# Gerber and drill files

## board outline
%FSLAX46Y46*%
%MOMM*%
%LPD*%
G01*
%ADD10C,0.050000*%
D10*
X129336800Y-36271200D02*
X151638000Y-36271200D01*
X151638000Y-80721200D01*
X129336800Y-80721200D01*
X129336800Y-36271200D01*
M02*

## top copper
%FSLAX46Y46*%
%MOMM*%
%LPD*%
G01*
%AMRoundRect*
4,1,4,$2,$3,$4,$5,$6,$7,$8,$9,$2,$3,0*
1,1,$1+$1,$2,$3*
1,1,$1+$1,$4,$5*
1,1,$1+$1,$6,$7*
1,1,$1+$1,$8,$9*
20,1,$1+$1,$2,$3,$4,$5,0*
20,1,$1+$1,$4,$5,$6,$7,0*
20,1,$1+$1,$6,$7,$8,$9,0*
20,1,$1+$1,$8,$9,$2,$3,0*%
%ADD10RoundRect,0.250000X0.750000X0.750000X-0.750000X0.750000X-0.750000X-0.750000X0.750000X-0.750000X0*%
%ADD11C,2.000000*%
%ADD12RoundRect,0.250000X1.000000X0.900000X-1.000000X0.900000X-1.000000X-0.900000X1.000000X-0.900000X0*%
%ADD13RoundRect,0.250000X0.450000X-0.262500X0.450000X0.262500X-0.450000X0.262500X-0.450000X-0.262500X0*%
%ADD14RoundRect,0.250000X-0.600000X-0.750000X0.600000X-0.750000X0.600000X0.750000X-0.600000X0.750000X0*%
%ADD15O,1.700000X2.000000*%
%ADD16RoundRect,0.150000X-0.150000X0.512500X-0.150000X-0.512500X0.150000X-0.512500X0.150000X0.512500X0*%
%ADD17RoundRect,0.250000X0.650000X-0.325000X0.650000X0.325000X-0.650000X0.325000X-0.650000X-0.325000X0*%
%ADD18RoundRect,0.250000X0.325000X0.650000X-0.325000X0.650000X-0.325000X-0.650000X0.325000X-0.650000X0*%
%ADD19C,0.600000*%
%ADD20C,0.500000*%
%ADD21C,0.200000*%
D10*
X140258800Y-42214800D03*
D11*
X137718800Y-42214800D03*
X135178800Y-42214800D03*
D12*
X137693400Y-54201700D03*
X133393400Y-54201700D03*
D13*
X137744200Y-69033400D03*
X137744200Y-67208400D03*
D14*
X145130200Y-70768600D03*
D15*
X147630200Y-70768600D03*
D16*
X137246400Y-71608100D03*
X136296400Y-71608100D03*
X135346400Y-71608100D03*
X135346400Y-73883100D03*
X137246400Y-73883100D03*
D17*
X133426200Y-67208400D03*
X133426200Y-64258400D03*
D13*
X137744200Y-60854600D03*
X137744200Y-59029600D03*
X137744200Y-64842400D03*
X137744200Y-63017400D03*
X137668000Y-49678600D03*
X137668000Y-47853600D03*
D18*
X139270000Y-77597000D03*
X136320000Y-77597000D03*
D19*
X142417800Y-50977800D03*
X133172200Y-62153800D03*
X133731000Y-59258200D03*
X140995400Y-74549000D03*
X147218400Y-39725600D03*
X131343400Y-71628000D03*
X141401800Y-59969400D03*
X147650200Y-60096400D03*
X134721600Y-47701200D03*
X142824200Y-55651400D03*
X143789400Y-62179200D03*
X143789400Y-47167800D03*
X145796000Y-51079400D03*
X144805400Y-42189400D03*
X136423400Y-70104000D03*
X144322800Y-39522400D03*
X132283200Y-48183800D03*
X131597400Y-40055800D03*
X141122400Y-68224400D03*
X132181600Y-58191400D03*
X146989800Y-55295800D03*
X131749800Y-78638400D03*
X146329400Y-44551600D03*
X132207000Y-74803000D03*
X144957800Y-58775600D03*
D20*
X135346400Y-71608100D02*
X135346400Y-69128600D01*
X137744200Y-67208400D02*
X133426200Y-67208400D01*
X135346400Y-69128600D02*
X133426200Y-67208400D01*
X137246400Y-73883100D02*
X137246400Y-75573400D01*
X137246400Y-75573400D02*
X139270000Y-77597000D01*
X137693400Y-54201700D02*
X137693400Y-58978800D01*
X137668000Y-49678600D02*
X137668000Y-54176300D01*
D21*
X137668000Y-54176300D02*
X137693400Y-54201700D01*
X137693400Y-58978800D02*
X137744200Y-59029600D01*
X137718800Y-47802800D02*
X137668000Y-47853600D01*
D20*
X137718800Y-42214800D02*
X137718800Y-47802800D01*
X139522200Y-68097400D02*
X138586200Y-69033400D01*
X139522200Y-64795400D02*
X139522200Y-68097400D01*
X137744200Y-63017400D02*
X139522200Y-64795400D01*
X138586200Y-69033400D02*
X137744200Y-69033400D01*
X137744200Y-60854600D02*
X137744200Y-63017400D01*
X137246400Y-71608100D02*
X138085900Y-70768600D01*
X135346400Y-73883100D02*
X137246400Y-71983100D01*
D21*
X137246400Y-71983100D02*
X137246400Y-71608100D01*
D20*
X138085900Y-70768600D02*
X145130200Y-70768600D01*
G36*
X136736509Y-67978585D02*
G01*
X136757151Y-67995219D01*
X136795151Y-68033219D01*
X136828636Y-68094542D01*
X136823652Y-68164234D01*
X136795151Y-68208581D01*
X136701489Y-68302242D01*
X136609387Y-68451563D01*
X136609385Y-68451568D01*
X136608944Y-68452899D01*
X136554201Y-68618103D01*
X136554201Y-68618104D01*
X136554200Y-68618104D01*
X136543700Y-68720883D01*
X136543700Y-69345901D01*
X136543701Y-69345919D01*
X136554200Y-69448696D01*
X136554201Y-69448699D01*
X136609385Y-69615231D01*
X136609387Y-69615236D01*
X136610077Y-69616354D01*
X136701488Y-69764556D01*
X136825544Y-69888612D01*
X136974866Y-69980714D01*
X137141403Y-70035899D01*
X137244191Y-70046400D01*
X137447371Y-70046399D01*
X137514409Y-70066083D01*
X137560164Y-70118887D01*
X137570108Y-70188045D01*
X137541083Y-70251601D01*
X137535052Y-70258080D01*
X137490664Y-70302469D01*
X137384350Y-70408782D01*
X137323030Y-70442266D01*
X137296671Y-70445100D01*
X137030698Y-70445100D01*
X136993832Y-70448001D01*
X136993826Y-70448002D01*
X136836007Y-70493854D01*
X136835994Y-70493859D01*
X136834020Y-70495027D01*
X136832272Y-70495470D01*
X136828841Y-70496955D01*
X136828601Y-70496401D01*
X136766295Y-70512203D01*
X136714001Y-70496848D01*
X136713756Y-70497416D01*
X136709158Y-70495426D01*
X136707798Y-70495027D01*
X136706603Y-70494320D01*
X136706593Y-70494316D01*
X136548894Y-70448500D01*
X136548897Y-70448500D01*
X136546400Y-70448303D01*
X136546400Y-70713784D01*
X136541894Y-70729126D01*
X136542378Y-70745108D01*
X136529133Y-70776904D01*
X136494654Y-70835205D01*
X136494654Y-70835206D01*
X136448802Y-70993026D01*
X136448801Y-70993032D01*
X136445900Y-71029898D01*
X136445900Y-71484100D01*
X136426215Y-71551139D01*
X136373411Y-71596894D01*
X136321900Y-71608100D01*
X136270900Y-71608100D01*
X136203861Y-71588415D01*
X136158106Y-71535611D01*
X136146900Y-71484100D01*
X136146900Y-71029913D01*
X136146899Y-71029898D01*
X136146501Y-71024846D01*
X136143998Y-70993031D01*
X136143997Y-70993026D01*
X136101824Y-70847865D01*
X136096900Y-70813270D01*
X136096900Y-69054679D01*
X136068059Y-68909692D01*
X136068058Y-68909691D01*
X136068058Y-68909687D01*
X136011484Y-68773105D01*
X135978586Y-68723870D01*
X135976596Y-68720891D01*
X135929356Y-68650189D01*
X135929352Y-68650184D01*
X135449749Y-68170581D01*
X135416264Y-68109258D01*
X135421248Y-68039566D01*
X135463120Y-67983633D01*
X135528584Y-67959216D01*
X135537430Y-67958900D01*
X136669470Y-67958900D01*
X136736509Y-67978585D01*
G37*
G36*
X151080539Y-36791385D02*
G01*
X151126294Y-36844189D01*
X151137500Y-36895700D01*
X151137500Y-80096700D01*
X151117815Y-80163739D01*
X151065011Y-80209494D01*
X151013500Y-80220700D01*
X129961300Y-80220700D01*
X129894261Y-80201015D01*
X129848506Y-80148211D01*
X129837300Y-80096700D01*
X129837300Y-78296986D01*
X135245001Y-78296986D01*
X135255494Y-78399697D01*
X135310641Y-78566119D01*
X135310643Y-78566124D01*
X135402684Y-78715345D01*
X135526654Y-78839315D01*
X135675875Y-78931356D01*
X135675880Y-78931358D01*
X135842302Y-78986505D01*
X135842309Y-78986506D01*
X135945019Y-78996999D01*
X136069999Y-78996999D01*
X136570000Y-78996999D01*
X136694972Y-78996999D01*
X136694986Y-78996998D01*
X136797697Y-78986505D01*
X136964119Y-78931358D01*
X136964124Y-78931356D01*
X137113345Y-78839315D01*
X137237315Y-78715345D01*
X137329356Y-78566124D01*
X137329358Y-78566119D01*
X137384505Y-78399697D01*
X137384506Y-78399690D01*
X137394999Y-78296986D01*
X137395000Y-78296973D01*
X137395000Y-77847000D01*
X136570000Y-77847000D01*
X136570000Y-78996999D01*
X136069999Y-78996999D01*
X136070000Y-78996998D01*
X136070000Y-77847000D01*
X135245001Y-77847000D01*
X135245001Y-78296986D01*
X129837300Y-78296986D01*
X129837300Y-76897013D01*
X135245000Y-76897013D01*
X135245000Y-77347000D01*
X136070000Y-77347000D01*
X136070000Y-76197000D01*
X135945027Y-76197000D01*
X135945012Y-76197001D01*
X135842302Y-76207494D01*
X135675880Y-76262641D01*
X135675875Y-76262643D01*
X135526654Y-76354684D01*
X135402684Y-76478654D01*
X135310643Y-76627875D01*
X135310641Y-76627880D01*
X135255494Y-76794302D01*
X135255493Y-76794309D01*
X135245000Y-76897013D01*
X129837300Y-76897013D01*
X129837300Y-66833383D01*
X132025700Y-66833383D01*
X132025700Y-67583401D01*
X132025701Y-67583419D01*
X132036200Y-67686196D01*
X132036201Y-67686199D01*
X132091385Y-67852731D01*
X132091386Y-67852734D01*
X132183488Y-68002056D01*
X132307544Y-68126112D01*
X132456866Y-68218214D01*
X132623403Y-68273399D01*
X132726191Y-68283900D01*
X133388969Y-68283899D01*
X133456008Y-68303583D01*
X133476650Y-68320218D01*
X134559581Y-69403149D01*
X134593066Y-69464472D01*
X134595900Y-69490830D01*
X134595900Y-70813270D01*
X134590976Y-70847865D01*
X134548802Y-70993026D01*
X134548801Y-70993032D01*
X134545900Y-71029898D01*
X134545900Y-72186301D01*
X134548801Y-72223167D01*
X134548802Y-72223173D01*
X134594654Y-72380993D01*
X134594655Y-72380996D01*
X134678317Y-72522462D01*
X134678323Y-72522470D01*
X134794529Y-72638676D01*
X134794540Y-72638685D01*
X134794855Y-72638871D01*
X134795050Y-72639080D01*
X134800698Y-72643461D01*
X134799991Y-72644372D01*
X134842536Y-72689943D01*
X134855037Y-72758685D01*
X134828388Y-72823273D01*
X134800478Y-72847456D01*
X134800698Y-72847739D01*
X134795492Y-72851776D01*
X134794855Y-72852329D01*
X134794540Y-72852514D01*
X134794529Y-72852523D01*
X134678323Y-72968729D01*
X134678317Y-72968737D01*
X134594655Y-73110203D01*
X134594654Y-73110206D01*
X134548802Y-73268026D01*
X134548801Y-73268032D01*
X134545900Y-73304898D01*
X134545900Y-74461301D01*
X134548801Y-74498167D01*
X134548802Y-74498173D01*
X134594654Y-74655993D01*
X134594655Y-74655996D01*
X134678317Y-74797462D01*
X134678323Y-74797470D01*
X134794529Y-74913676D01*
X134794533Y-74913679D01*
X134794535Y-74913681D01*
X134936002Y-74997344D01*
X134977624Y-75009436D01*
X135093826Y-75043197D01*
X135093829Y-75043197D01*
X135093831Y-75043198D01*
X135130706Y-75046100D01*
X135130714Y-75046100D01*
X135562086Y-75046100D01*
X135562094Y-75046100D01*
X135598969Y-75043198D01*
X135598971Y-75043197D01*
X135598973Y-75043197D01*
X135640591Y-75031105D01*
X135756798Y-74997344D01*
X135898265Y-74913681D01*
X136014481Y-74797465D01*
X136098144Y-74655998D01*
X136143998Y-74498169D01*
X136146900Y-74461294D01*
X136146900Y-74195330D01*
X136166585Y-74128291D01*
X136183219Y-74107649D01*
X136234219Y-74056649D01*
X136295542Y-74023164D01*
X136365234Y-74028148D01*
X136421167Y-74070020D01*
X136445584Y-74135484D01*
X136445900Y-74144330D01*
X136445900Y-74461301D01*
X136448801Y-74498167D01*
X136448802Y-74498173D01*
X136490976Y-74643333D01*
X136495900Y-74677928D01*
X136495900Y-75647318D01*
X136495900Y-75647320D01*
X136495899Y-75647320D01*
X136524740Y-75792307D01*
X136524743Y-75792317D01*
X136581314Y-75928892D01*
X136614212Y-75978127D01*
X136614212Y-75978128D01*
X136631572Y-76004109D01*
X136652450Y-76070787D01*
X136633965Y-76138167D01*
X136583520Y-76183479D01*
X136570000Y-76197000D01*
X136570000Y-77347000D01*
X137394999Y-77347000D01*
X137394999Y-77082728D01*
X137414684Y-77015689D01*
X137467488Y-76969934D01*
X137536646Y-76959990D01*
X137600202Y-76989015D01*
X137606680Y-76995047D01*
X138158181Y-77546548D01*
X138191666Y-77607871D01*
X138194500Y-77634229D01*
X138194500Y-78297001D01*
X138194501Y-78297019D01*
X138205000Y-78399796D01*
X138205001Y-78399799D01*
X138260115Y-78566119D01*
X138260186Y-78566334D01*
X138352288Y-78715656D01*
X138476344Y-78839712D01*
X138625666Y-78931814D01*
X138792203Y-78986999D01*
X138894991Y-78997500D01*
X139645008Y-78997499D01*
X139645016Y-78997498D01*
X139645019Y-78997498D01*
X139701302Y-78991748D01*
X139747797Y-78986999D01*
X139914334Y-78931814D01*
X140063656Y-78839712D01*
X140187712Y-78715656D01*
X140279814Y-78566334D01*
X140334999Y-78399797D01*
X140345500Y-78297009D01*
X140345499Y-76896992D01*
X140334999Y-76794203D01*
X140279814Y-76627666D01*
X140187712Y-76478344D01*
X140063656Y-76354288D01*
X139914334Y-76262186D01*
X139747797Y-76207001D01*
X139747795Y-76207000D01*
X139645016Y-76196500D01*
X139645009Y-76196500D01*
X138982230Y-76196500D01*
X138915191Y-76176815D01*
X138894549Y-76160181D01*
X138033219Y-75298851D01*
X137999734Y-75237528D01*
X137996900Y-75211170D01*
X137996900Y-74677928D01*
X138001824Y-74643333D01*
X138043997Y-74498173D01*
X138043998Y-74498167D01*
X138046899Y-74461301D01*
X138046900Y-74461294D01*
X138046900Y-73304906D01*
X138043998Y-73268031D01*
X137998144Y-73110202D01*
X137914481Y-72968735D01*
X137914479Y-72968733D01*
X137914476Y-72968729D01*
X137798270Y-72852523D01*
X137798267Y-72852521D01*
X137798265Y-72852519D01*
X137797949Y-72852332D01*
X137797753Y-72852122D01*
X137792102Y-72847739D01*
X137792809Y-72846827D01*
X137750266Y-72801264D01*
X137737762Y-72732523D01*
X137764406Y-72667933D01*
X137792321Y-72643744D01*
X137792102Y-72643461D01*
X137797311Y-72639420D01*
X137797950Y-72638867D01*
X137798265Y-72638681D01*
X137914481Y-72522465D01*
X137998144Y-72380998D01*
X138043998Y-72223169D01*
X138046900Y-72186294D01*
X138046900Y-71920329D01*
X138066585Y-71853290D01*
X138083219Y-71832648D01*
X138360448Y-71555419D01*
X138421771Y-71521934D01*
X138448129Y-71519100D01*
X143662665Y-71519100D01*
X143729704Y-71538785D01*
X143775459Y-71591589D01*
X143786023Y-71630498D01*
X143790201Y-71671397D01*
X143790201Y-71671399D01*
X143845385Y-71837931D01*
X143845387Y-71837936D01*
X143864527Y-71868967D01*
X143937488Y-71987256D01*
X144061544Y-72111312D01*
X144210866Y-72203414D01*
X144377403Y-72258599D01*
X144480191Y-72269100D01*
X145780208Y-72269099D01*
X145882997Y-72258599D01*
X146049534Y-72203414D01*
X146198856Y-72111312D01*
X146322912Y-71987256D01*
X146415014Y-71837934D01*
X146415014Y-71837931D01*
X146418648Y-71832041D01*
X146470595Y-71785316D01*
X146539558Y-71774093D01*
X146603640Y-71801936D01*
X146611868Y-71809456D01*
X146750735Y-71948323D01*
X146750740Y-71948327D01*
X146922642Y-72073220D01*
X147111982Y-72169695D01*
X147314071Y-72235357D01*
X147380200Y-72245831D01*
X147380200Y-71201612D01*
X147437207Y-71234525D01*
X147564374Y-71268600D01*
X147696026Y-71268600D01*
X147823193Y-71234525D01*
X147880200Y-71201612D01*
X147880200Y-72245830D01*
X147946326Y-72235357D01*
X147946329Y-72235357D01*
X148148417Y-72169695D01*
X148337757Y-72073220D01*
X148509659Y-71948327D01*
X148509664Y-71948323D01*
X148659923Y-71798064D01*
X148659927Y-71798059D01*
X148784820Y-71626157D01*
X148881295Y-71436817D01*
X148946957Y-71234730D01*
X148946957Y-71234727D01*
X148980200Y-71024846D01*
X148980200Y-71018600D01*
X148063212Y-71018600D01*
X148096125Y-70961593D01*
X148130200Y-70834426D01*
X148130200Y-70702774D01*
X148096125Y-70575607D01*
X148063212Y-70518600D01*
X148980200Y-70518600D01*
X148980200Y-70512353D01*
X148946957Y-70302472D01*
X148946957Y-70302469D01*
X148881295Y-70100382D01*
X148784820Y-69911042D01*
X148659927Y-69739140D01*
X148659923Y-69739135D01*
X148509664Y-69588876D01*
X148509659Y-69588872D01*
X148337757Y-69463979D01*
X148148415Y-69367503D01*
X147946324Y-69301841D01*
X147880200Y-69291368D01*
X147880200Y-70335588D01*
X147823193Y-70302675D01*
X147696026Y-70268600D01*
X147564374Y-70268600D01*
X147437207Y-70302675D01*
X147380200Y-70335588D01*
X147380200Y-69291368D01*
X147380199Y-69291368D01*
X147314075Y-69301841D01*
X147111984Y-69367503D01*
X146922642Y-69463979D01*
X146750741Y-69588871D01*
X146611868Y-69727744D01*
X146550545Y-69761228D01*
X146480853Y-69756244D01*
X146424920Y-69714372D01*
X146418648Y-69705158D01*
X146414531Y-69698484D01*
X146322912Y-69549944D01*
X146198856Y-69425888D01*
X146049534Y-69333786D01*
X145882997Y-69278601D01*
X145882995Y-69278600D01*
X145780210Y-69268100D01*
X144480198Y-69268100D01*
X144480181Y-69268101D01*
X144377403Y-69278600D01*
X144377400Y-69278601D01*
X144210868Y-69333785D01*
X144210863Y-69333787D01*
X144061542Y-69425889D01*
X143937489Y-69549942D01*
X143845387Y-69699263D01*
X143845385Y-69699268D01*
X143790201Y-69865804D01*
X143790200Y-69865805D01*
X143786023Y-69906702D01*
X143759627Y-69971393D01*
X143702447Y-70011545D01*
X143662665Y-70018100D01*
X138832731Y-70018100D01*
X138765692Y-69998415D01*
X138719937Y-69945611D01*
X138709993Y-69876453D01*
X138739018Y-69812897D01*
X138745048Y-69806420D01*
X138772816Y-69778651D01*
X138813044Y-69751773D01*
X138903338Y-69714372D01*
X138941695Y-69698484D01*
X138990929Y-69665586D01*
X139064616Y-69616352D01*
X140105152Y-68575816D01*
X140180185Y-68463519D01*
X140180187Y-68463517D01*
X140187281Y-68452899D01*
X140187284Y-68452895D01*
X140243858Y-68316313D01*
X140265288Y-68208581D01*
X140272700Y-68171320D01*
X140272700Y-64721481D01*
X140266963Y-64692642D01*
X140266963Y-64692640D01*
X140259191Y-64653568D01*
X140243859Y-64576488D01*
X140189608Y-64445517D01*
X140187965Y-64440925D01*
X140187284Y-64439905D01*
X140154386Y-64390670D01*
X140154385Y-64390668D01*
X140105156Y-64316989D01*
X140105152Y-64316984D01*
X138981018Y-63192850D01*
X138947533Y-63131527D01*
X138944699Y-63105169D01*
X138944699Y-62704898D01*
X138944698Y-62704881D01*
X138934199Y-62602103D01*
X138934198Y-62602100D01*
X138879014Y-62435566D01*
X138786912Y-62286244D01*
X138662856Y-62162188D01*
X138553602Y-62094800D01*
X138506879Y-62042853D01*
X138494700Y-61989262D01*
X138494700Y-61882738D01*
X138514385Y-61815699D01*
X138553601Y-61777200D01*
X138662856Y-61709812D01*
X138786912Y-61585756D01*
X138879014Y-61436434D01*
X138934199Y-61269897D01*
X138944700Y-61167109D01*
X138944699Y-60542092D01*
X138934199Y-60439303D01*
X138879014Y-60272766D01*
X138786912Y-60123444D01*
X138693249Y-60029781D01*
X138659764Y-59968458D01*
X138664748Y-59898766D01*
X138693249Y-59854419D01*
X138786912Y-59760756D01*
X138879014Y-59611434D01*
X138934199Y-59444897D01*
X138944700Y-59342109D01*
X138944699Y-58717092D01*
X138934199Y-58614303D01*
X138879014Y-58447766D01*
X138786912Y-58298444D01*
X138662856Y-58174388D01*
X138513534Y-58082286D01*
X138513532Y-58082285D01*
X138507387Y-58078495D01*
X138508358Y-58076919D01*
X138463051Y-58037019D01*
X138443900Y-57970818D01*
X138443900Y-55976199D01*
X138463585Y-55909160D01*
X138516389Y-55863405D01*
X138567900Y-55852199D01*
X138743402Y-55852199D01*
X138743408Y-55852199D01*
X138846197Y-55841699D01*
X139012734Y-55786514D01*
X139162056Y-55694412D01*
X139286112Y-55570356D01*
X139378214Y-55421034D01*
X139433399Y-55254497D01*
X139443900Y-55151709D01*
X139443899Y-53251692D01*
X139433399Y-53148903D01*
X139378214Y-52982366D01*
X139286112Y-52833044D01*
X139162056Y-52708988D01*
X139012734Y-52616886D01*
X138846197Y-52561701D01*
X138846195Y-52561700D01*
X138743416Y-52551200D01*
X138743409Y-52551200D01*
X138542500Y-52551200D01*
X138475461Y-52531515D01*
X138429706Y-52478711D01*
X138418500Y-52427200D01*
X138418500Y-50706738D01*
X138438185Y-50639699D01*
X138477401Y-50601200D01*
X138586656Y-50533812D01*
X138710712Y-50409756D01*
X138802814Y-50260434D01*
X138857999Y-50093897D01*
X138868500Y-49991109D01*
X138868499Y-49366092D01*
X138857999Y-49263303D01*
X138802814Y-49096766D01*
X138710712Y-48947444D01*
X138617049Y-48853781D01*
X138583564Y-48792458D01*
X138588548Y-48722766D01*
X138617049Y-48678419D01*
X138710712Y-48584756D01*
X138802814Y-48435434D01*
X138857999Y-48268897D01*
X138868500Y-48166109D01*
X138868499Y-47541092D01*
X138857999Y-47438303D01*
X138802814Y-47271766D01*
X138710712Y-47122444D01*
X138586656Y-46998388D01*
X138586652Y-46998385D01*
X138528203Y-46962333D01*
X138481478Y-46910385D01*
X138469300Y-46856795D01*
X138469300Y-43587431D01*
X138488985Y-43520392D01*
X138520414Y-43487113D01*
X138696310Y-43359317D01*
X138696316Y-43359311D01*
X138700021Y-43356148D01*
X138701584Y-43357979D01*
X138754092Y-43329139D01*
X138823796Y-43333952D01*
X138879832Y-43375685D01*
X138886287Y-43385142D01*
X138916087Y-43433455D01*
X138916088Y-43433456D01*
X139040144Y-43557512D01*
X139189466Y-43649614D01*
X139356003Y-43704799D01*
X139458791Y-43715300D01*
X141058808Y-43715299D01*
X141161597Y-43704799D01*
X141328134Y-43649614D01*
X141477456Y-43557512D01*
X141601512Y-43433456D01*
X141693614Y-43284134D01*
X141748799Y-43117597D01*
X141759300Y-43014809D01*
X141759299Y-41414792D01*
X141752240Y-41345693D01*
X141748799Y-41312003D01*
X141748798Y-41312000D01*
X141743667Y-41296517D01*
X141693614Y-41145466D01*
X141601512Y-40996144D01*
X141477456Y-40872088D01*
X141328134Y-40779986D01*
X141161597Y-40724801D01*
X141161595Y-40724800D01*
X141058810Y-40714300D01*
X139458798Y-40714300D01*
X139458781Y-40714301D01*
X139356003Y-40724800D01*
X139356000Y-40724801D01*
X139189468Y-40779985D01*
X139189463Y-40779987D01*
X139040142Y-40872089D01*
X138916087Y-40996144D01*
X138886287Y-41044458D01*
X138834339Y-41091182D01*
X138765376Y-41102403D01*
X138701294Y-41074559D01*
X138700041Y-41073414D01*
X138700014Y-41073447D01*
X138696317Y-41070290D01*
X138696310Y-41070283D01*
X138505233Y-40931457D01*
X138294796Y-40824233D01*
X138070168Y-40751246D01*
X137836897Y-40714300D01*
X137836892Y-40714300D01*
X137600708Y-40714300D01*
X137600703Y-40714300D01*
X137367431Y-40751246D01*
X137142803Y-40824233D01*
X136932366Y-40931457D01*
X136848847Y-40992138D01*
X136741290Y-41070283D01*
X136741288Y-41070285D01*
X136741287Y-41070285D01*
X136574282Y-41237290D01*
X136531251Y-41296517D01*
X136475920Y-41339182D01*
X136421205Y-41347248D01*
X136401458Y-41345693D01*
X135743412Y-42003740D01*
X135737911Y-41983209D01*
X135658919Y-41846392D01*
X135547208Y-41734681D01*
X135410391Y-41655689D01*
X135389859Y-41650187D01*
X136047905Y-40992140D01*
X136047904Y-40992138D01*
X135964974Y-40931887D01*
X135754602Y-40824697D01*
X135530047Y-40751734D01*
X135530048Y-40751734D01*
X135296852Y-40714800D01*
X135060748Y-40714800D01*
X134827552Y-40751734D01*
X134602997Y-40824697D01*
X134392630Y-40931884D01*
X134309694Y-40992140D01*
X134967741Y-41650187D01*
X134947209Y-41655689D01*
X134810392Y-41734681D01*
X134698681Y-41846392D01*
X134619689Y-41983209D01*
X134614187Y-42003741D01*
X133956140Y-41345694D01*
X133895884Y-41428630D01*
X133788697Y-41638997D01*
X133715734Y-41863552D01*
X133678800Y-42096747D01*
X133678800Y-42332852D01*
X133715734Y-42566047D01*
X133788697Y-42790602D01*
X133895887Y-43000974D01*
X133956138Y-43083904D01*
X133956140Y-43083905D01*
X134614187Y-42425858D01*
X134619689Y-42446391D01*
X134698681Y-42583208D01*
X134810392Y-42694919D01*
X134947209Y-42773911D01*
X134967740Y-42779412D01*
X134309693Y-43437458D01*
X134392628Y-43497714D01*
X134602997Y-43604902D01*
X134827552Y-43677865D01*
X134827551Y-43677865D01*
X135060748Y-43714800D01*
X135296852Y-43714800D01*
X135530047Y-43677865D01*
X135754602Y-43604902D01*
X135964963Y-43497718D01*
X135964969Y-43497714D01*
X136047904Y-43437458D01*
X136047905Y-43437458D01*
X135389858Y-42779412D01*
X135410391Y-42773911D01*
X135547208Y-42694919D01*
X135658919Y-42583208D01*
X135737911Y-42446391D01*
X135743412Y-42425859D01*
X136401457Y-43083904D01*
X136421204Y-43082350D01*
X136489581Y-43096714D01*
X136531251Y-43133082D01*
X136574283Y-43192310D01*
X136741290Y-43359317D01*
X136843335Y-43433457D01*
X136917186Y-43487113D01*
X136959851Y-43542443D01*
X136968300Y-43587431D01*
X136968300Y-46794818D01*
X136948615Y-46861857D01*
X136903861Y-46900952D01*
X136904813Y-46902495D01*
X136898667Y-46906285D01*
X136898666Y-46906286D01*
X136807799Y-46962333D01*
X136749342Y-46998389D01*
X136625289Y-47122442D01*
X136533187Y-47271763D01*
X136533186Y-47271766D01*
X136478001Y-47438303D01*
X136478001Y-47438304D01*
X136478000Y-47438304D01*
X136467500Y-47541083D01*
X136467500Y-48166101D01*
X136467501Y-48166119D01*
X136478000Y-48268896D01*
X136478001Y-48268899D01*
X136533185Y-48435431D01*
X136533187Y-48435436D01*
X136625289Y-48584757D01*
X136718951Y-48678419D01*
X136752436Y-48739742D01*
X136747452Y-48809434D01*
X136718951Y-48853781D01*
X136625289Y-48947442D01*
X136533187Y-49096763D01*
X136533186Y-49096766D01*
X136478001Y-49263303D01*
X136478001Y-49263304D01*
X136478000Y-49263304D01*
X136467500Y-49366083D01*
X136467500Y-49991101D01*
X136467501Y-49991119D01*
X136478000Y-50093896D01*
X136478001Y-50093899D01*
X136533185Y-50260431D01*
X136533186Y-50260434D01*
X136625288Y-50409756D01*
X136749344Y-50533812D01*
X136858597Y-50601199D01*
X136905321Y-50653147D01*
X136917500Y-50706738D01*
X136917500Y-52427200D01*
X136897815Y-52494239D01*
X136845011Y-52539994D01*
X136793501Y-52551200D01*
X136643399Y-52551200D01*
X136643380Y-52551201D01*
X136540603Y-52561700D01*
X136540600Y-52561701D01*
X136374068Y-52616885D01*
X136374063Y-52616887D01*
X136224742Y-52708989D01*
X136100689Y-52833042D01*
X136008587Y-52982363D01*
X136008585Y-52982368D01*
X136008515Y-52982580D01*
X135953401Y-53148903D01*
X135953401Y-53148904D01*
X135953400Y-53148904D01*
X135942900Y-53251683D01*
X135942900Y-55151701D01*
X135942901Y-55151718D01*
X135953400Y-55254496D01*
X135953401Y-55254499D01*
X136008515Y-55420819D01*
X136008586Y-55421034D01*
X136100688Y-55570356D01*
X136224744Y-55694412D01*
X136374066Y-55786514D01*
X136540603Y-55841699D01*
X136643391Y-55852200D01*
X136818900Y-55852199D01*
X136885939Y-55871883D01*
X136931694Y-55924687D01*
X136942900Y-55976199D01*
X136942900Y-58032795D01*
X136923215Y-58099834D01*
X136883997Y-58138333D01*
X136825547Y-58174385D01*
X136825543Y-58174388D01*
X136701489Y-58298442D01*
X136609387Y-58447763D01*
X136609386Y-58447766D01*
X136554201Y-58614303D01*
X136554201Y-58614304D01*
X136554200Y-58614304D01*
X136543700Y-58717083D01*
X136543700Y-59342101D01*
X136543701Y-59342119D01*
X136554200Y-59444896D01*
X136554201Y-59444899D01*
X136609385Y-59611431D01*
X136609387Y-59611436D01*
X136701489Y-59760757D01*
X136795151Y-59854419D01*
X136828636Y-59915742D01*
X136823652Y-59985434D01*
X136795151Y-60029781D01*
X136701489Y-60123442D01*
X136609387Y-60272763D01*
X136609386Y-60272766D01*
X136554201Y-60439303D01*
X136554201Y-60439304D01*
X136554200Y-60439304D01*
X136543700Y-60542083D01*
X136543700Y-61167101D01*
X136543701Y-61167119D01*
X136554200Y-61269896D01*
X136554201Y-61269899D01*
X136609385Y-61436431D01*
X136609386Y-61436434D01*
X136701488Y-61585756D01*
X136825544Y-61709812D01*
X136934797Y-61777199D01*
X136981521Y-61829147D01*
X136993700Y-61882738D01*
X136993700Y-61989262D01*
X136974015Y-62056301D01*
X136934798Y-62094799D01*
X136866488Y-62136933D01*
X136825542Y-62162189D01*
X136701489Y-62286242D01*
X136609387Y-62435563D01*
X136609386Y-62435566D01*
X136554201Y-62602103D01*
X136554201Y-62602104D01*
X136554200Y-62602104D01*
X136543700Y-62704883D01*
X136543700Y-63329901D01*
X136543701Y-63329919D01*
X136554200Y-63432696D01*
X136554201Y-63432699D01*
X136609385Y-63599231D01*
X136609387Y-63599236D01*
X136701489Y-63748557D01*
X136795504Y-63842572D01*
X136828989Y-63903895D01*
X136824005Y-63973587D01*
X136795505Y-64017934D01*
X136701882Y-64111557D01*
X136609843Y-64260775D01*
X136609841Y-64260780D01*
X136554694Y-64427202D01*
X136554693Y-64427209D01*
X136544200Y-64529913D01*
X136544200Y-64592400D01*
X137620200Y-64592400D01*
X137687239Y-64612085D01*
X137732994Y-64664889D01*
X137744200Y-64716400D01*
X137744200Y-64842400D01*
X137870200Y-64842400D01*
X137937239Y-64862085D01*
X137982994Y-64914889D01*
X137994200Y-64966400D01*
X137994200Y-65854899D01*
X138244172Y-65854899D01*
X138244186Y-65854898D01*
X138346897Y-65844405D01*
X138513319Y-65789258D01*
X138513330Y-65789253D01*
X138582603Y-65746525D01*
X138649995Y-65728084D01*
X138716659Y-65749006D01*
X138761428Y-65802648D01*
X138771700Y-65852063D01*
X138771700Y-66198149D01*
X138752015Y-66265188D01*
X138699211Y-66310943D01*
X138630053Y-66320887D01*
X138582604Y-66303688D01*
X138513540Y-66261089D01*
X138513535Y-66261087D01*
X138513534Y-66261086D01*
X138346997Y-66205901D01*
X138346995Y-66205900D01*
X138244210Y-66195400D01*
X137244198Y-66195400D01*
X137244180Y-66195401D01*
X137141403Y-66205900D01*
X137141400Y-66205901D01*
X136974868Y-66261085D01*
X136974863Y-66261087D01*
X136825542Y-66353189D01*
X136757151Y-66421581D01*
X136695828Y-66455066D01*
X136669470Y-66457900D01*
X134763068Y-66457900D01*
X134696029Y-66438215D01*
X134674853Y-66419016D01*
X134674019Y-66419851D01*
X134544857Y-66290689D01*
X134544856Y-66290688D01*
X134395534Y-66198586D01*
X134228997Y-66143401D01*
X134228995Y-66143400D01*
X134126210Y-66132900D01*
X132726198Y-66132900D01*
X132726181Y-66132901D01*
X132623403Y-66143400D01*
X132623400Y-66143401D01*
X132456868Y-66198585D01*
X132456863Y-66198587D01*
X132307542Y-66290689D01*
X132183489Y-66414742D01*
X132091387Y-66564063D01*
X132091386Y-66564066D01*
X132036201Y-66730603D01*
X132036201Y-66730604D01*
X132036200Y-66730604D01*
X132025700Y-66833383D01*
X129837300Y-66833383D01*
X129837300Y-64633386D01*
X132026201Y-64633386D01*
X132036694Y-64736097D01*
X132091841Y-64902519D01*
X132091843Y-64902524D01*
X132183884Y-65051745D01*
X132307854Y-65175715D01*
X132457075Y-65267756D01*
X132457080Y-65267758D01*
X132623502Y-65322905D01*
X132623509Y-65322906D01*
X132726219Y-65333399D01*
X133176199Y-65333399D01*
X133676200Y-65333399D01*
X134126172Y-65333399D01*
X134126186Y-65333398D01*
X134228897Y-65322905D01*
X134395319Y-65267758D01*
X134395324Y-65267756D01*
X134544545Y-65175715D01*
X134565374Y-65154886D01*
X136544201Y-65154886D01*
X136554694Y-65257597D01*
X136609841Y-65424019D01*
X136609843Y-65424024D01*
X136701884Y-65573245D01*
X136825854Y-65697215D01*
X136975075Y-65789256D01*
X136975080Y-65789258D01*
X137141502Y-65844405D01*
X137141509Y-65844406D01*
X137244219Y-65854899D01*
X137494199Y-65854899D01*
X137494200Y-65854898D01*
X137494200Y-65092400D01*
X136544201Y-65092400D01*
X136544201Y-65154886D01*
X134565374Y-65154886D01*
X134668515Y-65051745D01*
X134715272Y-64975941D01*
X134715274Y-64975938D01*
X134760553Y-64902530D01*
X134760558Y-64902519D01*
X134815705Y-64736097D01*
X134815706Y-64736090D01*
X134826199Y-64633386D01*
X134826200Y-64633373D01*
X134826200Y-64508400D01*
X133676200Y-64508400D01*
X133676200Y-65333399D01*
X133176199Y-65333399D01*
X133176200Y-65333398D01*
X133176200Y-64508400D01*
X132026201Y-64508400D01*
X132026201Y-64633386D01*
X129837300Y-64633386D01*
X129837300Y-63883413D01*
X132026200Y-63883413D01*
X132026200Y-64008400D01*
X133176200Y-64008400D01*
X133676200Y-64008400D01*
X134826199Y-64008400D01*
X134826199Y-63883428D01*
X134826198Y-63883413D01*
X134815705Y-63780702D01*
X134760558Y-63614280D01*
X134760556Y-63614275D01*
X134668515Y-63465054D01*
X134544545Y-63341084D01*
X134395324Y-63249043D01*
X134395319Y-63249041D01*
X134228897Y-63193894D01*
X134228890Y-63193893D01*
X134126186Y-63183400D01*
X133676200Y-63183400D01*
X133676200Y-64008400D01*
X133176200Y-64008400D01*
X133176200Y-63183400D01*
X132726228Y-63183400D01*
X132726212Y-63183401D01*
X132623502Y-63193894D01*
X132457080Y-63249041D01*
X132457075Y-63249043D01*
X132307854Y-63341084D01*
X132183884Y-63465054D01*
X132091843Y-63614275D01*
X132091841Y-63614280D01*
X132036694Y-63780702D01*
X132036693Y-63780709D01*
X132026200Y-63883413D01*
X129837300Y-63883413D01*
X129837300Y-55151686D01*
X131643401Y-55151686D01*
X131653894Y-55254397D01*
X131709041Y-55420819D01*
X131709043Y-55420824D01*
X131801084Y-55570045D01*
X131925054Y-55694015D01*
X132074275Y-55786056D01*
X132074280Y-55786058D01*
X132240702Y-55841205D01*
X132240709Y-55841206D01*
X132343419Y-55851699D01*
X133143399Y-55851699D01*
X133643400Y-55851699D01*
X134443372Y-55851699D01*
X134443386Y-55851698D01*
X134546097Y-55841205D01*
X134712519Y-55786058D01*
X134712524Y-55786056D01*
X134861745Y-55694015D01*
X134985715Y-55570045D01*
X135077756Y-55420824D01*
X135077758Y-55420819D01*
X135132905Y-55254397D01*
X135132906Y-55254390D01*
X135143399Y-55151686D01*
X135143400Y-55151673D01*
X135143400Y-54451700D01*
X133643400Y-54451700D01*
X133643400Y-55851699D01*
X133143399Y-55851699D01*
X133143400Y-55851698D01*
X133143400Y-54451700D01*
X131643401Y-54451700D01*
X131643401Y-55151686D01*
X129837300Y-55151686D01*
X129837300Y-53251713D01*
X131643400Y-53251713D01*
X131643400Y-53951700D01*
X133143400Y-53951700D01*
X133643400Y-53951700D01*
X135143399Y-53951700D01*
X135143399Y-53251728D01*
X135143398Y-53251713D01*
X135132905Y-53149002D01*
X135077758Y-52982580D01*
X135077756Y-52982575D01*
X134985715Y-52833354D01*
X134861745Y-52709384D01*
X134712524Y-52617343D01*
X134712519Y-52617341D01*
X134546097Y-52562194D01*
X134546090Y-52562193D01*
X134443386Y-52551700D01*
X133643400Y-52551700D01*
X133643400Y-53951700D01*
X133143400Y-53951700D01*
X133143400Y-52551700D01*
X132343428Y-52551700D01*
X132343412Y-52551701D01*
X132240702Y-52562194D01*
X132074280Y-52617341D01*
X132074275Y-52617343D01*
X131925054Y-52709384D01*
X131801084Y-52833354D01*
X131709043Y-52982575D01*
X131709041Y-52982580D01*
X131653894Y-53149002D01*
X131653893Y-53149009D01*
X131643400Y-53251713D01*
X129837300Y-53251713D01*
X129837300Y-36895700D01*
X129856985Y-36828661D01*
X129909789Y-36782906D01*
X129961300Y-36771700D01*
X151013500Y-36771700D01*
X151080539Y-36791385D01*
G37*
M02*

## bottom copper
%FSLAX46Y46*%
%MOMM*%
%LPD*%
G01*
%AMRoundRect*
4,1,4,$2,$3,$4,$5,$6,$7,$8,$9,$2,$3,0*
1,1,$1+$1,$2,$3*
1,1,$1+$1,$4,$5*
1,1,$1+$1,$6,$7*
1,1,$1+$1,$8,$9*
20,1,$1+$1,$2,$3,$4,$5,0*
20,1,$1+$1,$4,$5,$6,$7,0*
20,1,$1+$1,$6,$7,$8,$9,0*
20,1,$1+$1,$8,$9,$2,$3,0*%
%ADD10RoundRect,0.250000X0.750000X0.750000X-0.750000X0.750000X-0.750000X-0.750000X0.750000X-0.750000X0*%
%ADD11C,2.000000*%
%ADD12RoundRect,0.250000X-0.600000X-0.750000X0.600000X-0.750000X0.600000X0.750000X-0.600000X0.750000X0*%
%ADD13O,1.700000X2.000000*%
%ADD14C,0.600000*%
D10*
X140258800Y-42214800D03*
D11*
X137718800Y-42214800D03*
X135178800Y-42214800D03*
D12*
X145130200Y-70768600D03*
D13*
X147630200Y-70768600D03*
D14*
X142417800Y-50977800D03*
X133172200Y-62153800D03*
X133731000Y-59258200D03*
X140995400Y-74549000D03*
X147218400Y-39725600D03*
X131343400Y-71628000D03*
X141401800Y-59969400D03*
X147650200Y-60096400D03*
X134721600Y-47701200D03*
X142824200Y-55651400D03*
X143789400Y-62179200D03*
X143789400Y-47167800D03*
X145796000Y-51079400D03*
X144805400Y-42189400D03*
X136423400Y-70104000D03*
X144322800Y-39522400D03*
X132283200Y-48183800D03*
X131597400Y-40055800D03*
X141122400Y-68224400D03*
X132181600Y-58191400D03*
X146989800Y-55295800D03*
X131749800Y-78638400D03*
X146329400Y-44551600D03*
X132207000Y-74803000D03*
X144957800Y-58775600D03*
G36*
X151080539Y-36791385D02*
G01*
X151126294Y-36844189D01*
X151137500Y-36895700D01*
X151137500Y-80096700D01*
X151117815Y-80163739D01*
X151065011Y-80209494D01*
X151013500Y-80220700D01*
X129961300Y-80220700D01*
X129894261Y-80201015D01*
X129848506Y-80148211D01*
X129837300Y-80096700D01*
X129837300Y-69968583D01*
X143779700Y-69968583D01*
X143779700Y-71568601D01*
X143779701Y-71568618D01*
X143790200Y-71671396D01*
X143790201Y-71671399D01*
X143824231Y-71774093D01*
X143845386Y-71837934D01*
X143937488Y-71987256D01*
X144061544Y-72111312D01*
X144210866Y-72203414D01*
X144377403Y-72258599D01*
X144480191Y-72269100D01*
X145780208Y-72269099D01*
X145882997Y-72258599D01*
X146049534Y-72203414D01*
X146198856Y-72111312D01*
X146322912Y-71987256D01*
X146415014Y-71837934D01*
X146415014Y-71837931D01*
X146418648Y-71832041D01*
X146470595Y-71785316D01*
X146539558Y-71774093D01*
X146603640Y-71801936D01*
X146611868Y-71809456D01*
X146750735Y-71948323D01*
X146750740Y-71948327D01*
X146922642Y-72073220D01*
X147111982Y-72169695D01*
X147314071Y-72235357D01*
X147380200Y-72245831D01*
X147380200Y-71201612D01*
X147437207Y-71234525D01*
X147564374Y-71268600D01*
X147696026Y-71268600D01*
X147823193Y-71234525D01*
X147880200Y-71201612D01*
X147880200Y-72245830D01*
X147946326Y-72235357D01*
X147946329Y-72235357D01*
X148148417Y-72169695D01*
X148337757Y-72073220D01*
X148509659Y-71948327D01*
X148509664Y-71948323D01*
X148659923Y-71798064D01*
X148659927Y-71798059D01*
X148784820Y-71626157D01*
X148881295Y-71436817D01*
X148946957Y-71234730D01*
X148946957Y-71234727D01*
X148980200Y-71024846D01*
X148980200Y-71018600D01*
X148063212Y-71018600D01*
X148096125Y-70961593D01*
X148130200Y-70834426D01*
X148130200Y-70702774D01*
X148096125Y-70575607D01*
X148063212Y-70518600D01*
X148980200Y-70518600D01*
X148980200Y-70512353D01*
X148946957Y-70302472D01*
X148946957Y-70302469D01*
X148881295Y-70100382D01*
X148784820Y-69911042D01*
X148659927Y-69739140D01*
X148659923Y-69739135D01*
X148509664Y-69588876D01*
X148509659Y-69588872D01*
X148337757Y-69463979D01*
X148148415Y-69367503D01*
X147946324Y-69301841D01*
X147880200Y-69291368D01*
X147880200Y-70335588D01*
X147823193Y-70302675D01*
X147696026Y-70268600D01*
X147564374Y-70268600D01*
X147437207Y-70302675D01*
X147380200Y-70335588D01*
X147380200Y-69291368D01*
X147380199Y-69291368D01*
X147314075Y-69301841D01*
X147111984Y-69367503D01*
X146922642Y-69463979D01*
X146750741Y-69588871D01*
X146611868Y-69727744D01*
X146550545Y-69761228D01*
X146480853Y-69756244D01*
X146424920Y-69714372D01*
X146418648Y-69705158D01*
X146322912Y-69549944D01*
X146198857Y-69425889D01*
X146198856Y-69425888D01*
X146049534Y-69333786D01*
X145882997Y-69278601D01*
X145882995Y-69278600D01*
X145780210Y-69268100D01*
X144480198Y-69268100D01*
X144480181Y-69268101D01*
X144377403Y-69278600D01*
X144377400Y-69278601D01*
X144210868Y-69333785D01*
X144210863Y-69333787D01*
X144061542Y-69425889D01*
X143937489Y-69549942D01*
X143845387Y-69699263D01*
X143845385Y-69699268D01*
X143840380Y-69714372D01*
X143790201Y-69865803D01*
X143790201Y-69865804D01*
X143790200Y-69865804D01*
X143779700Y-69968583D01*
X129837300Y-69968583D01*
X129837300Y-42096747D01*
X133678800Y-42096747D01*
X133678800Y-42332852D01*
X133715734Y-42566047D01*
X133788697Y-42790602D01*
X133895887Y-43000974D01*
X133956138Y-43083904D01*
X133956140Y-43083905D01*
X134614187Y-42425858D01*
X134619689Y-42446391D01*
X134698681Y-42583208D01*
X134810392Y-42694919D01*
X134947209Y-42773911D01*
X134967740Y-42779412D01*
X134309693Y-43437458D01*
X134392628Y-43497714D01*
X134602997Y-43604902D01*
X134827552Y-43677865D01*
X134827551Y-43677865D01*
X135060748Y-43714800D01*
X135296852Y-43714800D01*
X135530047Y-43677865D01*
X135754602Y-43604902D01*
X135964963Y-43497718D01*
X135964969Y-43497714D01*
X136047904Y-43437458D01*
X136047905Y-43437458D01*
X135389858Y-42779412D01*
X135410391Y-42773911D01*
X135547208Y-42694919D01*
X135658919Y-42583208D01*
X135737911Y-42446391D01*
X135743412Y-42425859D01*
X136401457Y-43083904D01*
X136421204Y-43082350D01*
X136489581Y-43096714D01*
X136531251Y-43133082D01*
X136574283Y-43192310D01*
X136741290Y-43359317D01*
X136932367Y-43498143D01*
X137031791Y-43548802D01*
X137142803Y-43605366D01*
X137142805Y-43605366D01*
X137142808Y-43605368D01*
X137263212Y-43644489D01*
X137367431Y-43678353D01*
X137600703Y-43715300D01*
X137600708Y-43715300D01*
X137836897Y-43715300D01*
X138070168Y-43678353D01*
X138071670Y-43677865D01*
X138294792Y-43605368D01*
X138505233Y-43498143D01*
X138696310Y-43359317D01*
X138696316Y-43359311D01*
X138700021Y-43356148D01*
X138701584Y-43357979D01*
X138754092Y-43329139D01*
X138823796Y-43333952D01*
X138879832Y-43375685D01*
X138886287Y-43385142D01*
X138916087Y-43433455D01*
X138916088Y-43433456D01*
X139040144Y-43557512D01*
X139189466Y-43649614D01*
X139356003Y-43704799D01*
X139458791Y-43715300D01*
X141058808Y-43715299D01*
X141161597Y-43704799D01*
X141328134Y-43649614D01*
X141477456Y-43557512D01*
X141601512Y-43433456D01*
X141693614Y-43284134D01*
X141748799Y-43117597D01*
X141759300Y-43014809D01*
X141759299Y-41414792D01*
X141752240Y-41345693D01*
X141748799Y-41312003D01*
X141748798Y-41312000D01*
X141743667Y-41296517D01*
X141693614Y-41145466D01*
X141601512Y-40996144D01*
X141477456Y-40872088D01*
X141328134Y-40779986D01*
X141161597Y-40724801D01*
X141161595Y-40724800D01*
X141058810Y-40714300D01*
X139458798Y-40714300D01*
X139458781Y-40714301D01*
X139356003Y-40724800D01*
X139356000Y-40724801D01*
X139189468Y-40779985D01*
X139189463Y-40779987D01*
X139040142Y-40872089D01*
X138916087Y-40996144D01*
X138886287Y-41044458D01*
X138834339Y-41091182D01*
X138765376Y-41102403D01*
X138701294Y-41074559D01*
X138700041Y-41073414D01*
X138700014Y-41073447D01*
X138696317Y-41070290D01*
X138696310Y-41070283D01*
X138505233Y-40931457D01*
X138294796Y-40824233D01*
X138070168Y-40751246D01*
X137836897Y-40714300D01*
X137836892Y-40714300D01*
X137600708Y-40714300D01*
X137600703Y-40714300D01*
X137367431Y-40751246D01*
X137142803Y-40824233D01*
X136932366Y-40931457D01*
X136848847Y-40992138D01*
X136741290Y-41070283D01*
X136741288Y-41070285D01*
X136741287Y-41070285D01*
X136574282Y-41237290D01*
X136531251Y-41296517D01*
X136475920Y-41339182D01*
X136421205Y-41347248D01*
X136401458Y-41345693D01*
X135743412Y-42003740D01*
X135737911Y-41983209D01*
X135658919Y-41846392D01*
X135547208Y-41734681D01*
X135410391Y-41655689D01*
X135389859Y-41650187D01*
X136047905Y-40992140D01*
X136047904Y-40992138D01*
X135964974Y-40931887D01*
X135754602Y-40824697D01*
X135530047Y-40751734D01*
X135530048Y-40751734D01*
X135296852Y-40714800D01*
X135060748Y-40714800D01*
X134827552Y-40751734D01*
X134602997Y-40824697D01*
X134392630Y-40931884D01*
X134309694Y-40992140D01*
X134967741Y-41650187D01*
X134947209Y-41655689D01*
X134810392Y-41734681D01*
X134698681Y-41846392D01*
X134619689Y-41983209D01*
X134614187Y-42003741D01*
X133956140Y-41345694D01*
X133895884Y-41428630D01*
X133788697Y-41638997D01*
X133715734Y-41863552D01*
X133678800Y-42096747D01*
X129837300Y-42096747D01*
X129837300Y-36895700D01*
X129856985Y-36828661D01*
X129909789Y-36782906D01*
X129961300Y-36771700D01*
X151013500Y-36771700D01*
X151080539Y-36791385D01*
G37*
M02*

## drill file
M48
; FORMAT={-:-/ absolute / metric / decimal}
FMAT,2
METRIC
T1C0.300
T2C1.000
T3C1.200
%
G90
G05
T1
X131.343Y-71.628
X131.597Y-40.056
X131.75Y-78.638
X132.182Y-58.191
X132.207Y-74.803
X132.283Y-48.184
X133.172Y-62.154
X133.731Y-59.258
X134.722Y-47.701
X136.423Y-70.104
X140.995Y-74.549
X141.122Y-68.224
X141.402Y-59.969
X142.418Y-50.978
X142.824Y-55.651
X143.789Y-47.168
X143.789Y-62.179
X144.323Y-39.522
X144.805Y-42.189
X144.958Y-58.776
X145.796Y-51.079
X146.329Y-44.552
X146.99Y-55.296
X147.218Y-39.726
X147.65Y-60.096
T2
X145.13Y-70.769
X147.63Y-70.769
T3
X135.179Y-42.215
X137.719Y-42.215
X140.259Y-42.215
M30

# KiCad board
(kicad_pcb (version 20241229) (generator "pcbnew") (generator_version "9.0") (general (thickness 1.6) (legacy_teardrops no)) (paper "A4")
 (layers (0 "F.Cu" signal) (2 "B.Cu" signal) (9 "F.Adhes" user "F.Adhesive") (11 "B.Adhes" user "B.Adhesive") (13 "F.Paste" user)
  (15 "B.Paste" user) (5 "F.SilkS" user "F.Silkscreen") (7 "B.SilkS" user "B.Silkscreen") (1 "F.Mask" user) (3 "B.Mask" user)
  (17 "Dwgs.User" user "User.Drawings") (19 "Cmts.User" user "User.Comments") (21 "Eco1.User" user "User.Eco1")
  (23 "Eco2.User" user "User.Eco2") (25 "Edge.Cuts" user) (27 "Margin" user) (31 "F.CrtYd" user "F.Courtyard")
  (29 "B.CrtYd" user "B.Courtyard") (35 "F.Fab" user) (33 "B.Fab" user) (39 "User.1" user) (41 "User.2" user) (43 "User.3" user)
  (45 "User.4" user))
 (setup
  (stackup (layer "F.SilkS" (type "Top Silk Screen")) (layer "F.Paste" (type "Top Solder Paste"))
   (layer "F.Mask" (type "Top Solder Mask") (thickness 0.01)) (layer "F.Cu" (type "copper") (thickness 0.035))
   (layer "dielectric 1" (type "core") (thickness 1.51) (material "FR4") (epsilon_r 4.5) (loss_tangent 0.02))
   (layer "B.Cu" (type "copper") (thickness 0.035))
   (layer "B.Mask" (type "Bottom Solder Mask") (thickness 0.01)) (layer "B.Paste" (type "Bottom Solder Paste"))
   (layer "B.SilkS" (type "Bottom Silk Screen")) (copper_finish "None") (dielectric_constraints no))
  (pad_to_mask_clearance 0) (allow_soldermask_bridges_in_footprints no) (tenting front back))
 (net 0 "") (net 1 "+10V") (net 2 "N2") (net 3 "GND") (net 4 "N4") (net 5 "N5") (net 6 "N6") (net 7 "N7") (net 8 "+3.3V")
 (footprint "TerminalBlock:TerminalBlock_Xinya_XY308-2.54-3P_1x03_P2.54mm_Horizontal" (layer "F.Cu") (at 140.2588 42.2148 180)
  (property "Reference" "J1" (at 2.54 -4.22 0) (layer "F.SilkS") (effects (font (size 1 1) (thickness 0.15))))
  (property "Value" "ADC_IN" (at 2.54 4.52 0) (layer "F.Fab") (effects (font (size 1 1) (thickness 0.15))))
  (pad "1" thru_hole roundrect (at 0 0 180) (size 2 2) (drill 1.2) (layers "*.Cu" "*.Mask") (remove_unused_layers no)
   (roundrect_rratio 0.125) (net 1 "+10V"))
  (pad "2" thru_hole circle (at 2.54 0 180) (size 2 2) (drill 1.2) (layers "*.Cu" "*.Mask") (remove_unused_layers no) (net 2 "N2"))
  (pad "3" thru_hole circle (at 5.08 0 180) (size 2 2) (drill 1.2) (layers "*.Cu" "*.Mask") (remove_unused_layers no) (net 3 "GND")))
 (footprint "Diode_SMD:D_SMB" (layer "F.Cu") (at 135.5434 54.2017 180)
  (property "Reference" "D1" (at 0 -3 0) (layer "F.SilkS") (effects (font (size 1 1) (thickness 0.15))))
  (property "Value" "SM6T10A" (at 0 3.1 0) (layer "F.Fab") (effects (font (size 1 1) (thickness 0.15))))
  (pad "1" smd roundrect (at -2.15 0 180) (size 2.5 2.3) (layers "F.Cu" "F.Mask" "F.Paste") (roundrect_rratio 0.1086956522) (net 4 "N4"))
  (pad "2" smd roundrect (at 2.15 0 180) (size 2.5 2.3) (layers "F.Cu" "F.Mask" "F.Paste") (roundrect_rratio 0.1086956522) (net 3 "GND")))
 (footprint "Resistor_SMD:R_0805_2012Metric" (layer "F.Cu") (at 137.7442 68.1209 90)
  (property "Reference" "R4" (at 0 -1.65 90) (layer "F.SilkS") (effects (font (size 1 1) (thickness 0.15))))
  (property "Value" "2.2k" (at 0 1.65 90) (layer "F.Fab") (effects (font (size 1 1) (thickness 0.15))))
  (pad "1" smd roundrect (at -0.9125 0 90) (size 1.025 1.4) (layers "F.Cu" "F.Mask" "F.Paste") (roundrect_rratio 0.243902) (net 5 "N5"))
  (pad "2" smd roundrect (at 0.9125 0 90) (size 1.025 1.4) (layers "F.Cu" "F.Mask" "F.Paste") (roundrect_rratio 0.243902) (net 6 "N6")))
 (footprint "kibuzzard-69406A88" (layer "F.Cu") (at 149.8346 46.2788 90)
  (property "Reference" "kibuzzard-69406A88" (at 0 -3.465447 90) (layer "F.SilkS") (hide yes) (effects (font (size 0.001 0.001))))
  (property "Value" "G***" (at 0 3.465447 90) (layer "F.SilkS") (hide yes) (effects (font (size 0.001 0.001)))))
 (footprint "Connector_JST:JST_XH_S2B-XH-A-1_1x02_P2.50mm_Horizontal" (layer "F.Cu") (at 145.1302 70.7686)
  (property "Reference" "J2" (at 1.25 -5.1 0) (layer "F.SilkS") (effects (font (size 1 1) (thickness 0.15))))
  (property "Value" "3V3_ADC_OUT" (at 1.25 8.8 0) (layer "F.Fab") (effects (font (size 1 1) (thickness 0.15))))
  (pad "1" thru_hole roundrect (at 0 0) (size 1.7 2) (drill 1) (layers "*.Cu" "*.Mask") (remove_unused_layers no)
   (roundrect_rratio 0.147059) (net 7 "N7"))
  (pad "2" thru_hole oval (at 2.5 0) (size 1.7 2) (drill 1) (layers "*.Cu" "*.Mask") (remove_unused_layers no) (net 3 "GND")))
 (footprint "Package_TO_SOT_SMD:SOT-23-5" (layer "F.Cu") (at 136.2964 72.7456 -90)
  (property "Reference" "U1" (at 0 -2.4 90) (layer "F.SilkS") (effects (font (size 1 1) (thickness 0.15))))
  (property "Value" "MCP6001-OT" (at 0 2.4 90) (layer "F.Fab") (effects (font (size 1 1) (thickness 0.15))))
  (pad "1" smd roundrect (at -1.1375 -0.95 270) (size 1.325 0.6) (layers "F.Cu" "F.Mask" "F.Paste") (roundrect_rratio 0.25) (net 7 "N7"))
  (pad "2" smd roundrect (at -1.1375 0 270) (size 1.325 0.6) (layers "F.Cu" "F.Mask" "F.Paste") (roundrect_rratio 0.25) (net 3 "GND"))
  (pad "3" smd roundrect (at -1.1375 0.95 270) (size 1.325 0.6) (layers "F.Cu" "F.Mask" "F.Paste") (roundrect_rratio 0.25) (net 6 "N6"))
  (pad "4" smd roundrect (at 1.1375 0.95 270) (size 1.325 0.6) (layers "F.Cu" "F.Mask" "F.Paste") (roundrect_rratio 0.25) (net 7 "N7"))
  (pad "5" smd roundrect (at 1.1375 -0.95 270) (size 1.325 0.6) (layers "F.Cu" "F.Mask" "F.Paste") (roundrect_rratio 0.25) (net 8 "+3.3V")))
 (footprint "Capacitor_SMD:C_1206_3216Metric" (layer "F.Cu") (at 133.4262 65.7334 90)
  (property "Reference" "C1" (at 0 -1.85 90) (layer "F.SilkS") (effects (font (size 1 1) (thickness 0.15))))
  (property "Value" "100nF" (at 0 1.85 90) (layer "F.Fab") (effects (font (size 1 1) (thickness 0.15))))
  (pad "1" smd roundrect (at -1.475 0 90) (size 1.15 1.8) (layers "F.Cu" "F.Mask" "F.Paste") (roundrect_rratio 0.217391) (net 6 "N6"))
  (pad "2" smd roundrect (at 1.475 0 90) (size 1.15 1.8) (layers "F.Cu" "F.Mask" "F.Paste") (roundrect_rratio 0.217391) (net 3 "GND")))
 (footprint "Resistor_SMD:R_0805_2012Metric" (layer "F.Cu") (at 137.7442 59.9421 90)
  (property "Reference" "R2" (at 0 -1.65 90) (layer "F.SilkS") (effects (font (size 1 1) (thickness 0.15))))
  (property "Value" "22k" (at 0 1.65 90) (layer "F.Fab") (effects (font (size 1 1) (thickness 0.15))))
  (pad "1" smd roundrect (at -0.9125 0 90) (size 1.025 1.4) (layers "F.Cu" "F.Mask" "F.Paste") (roundrect_rratio 0.243902) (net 5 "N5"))
  (pad "2" smd roundrect (at 0.9125 0 90) (size 1.025 1.4) (layers "F.Cu" "F.Mask" "F.Paste") (roundrect_rratio 0.243902) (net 4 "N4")))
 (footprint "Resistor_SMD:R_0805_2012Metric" (layer "F.Cu") (at 137.7442 63.9299 90)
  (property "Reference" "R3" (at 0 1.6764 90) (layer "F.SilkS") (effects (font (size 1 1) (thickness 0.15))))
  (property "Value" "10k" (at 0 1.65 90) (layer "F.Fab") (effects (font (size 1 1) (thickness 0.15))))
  (pad "1" smd roundrect (at -0.9125 0 90) (size 1.025 1.4) (layers "F.Cu" "F.Mask" "F.Paste") (roundrect_rratio 0.243902) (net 3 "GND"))
  (pad "2" smd roundrect (at 0.9125 0 90) (size 1.025 1.4) (layers "F.Cu" "F.Mask" "F.Paste") (roundrect_rratio 0.243902) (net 5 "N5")))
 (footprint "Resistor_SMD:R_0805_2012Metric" (layer "F.Cu") (at 137.668 48.7661 90)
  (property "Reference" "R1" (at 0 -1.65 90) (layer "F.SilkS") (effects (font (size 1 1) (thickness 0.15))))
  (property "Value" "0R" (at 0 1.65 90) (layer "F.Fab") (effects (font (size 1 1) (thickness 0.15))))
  (pad "1" smd roundrect (at -0.9125 0 90) (size 1.025 1.4) (layers "F.Cu" "F.Mask" "F.Paste") (roundrect_rratio 0.243902) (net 4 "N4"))
  (pad "2" smd roundrect (at 0.9125 0 90) (size 1.025 1.4) (layers "F.Cu" "F.Mask" "F.Paste") (roundrect_rratio 0.243902) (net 2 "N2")))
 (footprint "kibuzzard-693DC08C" (layer "F.Cu") (at 140.2842 37.2872 180)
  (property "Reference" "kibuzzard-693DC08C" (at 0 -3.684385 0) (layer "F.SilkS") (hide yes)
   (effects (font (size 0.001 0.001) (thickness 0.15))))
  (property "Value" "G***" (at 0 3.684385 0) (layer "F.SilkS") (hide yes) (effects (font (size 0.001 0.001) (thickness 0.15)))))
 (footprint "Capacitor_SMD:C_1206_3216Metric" (layer "F.Cu") (at 137.795 77.597 180)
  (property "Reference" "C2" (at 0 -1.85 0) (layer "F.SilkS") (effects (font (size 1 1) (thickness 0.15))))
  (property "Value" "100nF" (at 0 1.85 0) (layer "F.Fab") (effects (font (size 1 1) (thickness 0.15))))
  (pad "1" smd roundrect (at -1.475 0 180) (size 1.15 1.8) (layers "F.Cu" "F.Mask" "F.Paste") (roundrect_rratio 0.217391) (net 8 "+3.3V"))
  (pad "2" smd roundrect (at 1.475 0 180) (size 1.15 1.8) (layers "F.Cu" "F.Mask" "F.Paste") (roundrect_rratio 0.217391) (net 3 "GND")))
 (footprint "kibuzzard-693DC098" (layer "F.Cu") (at 137.9474 37.2364 180)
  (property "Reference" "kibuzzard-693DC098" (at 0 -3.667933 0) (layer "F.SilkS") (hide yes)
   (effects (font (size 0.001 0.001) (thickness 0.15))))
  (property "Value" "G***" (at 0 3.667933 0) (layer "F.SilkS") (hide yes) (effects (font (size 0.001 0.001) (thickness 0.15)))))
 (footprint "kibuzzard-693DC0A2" (layer "F.Cu") (at 135.2042 37.2364 180)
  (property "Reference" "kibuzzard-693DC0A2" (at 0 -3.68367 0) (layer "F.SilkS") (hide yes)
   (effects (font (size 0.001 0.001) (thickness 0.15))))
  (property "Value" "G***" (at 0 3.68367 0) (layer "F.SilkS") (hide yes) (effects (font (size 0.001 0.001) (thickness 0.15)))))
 (gr_rect (start 129.3368 36.2712) (end 151.638 80.7212) (stroke (width 0.05) (type default)) (fill no) (layer "Edge.Cuts"))
 (via (at 142.4178 50.9778) (size 0.6) (drill 0.3) (layers "F.Cu" "B.Cu") (free yes) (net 3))
 (via (at 133.1722 62.1538) (size 0.6) (drill 0.3) (layers "F.Cu" "B.Cu") (free yes) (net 3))
 (via (at 133.731 59.2582) (size 0.6) (drill 0.3) (layers "F.Cu" "B.Cu") (free yes) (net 3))
 (via (at 140.9954 74.549) (size 0.6) (drill 0.3) (layers "F.Cu" "B.Cu") (free yes) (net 3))
 (via (at 147.2184 39.7256) (size 0.6) (drill 0.3) (layers "F.Cu" "B.Cu") (free yes) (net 3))
 (via (at 131.3434 71.628) (size 0.6) (drill 0.3) (layers "F.Cu" "B.Cu") (free yes) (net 3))
 (via (at 141.4018 59.9694) (size 0.6) (drill 0.3) (layers "F.Cu" "B.Cu") (free yes) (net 3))
 (via (at 147.6502 60.0964) (size 0.6) (drill 0.3) (layers "F.Cu" "B.Cu") (free yes) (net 3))
 (via (at 134.7216 47.7012) (size 0.6) (drill 0.3) (layers "F.Cu" "B.Cu") (free yes) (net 3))
 (via (at 142.8242 55.6514) (size 0.6) (drill 0.3) (layers "F.Cu" "B.Cu") (free yes) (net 3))
 (via (at 143.7894 62.1792) (size 0.6) (drill 0.3) (layers "F.Cu" "B.Cu") (free yes) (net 3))
 (via (at 143.7894 47.1678) (size 0.6) (drill 0.3) (layers "F.Cu" "B.Cu") (free yes) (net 3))
 (via (at 145.796 51.0794) (size 0.6) (drill 0.3) (layers "F.Cu" "B.Cu") (free yes) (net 3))
 (via (at 144.8054 42.1894) (size 0.6) (drill 0.3) (layers "F.Cu" "B.Cu") (free yes) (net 3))
 (via (at 136.4234 70.104) (size 0.6) (drill 0.3) (layers "F.Cu" "B.Cu") (free yes) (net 3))
 (via (at 144.3228 39.5224) (size 0.6) (drill 0.3) (layers "F.Cu" "B.Cu") (free yes) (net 3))
 (via (at 132.2832 48.1838) (size 0.6) (drill 0.3) (layers "F.Cu" "B.Cu") (free yes) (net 3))
 (via (at 131.5974 40.0558) (size 0.6) (drill 0.3) (layers "F.Cu" "B.Cu") (free yes) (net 3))
 (via (at 141.1224 68.2244) (size 0.6) (drill 0.3) (layers "F.Cu" "B.Cu") (free yes) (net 3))
 (via (at 132.1816 58.1914) (size 0.6) (drill 0.3) (layers "F.Cu" "B.Cu") (free yes) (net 3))
 (via (at 146.9898 55.2958) (size 0.6) (drill 0.3) (layers "F.Cu" "B.Cu") (free yes) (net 3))
 (via (at 131.7498 78.6384) (size 0.6) (drill 0.3) (layers "F.Cu" "B.Cu") (free yes) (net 3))
 (via (at 146.3294 44.5516) (size 0.6) (drill 0.3) (layers "F.Cu" "B.Cu") (free yes) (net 3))
 (via (at 132.207 74.803) (size 0.6) (drill 0.3) (layers "F.Cu" "B.Cu") (free yes) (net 3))
 (via (at 144.9578 58.7756) (size 0.6) (drill 0.3) (layers "F.Cu" "B.Cu") (free yes) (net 3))
 (segment (start 135.3464 71.6081) (end 135.3464 69.1286) (width 0.5) (layer "F.Cu") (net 6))
 (segment (start 137.7442 67.2084) (end 133.4262 67.2084) (width 0.5) (layer "F.Cu") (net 6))
 (segment (start 135.3464 69.1286) (end 133.4262 67.2084) (width 0.5) (layer "F.Cu") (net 6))
 (segment (start 137.2464 73.8831) (end 137.2464 75.5734) (width 0.5) (layer "F.Cu") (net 8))
 (segment (start 137.2464 75.5734) (end 139.27 77.597) (width 0.5) (layer "F.Cu") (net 8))
 (segment (start 137.6934 54.2017) (end 137.6934 58.9788) (width 0.5) (layer "F.Cu") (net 4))
 (segment (start 137.668 49.6786) (end 137.668 54.1763) (width 0.5) (layer "F.Cu") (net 4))
 (segment (start 137.668 54.1763) (end 137.6934 54.2017) (width 0.2) (layer "F.Cu") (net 4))
 (segment (start 137.6934 58.9788) (end 137.7442 59.0296) (width 0.2) (layer "F.Cu") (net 4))
 (segment (start 137.7188 47.8028) (end 137.668 47.8536) (width 0.2) (layer "F.Cu") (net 2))
 (segment (start 137.7188 42.2148) (end 137.7188 47.8028) (width 0.5) (layer "F.Cu") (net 2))
 (segment (start 139.5222 68.0974) (end 138.5862 69.0334) (width 0.5) (layer "F.Cu") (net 5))
 (segment (start 139.5222 64.7954) (end 139.5222 68.0974) (width 0.5) (layer "F.Cu") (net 5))
 (segment (start 137.7442 63.0174) (end 139.5222 64.7954) (width 0.5) (layer "F.Cu") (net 5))
 (segment (start 138.5862 69.0334) (end 137.7442 69.0334) (width 0.5) (layer "F.Cu") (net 5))
 (segment (start 137.7442 60.8546) (end 137.7442 63.0174) (width 0.5) (layer "F.Cu") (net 5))
 (segment (start 137.2464 71.6081) (end 138.0859 70.7686) (width 0.5) (layer "F.Cu") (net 7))
 (segment (start 135.3464 73.8831) (end 137.2464 71.9831) (width 0.5) (layer "F.Cu") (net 7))
 (segment (start 137.2464 71.9831) (end 137.2464 71.6081) (width 0.2) (layer "F.Cu") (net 7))
 (segment (start 138.0859 70.7686) (end 145.1302 70.7686) (width 0.5) (layer "F.Cu") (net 7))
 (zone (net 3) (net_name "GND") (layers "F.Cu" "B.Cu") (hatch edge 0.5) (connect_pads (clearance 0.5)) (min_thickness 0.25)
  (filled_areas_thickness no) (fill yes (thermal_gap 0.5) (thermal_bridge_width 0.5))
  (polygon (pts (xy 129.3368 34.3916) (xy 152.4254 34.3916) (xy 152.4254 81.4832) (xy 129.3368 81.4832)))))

